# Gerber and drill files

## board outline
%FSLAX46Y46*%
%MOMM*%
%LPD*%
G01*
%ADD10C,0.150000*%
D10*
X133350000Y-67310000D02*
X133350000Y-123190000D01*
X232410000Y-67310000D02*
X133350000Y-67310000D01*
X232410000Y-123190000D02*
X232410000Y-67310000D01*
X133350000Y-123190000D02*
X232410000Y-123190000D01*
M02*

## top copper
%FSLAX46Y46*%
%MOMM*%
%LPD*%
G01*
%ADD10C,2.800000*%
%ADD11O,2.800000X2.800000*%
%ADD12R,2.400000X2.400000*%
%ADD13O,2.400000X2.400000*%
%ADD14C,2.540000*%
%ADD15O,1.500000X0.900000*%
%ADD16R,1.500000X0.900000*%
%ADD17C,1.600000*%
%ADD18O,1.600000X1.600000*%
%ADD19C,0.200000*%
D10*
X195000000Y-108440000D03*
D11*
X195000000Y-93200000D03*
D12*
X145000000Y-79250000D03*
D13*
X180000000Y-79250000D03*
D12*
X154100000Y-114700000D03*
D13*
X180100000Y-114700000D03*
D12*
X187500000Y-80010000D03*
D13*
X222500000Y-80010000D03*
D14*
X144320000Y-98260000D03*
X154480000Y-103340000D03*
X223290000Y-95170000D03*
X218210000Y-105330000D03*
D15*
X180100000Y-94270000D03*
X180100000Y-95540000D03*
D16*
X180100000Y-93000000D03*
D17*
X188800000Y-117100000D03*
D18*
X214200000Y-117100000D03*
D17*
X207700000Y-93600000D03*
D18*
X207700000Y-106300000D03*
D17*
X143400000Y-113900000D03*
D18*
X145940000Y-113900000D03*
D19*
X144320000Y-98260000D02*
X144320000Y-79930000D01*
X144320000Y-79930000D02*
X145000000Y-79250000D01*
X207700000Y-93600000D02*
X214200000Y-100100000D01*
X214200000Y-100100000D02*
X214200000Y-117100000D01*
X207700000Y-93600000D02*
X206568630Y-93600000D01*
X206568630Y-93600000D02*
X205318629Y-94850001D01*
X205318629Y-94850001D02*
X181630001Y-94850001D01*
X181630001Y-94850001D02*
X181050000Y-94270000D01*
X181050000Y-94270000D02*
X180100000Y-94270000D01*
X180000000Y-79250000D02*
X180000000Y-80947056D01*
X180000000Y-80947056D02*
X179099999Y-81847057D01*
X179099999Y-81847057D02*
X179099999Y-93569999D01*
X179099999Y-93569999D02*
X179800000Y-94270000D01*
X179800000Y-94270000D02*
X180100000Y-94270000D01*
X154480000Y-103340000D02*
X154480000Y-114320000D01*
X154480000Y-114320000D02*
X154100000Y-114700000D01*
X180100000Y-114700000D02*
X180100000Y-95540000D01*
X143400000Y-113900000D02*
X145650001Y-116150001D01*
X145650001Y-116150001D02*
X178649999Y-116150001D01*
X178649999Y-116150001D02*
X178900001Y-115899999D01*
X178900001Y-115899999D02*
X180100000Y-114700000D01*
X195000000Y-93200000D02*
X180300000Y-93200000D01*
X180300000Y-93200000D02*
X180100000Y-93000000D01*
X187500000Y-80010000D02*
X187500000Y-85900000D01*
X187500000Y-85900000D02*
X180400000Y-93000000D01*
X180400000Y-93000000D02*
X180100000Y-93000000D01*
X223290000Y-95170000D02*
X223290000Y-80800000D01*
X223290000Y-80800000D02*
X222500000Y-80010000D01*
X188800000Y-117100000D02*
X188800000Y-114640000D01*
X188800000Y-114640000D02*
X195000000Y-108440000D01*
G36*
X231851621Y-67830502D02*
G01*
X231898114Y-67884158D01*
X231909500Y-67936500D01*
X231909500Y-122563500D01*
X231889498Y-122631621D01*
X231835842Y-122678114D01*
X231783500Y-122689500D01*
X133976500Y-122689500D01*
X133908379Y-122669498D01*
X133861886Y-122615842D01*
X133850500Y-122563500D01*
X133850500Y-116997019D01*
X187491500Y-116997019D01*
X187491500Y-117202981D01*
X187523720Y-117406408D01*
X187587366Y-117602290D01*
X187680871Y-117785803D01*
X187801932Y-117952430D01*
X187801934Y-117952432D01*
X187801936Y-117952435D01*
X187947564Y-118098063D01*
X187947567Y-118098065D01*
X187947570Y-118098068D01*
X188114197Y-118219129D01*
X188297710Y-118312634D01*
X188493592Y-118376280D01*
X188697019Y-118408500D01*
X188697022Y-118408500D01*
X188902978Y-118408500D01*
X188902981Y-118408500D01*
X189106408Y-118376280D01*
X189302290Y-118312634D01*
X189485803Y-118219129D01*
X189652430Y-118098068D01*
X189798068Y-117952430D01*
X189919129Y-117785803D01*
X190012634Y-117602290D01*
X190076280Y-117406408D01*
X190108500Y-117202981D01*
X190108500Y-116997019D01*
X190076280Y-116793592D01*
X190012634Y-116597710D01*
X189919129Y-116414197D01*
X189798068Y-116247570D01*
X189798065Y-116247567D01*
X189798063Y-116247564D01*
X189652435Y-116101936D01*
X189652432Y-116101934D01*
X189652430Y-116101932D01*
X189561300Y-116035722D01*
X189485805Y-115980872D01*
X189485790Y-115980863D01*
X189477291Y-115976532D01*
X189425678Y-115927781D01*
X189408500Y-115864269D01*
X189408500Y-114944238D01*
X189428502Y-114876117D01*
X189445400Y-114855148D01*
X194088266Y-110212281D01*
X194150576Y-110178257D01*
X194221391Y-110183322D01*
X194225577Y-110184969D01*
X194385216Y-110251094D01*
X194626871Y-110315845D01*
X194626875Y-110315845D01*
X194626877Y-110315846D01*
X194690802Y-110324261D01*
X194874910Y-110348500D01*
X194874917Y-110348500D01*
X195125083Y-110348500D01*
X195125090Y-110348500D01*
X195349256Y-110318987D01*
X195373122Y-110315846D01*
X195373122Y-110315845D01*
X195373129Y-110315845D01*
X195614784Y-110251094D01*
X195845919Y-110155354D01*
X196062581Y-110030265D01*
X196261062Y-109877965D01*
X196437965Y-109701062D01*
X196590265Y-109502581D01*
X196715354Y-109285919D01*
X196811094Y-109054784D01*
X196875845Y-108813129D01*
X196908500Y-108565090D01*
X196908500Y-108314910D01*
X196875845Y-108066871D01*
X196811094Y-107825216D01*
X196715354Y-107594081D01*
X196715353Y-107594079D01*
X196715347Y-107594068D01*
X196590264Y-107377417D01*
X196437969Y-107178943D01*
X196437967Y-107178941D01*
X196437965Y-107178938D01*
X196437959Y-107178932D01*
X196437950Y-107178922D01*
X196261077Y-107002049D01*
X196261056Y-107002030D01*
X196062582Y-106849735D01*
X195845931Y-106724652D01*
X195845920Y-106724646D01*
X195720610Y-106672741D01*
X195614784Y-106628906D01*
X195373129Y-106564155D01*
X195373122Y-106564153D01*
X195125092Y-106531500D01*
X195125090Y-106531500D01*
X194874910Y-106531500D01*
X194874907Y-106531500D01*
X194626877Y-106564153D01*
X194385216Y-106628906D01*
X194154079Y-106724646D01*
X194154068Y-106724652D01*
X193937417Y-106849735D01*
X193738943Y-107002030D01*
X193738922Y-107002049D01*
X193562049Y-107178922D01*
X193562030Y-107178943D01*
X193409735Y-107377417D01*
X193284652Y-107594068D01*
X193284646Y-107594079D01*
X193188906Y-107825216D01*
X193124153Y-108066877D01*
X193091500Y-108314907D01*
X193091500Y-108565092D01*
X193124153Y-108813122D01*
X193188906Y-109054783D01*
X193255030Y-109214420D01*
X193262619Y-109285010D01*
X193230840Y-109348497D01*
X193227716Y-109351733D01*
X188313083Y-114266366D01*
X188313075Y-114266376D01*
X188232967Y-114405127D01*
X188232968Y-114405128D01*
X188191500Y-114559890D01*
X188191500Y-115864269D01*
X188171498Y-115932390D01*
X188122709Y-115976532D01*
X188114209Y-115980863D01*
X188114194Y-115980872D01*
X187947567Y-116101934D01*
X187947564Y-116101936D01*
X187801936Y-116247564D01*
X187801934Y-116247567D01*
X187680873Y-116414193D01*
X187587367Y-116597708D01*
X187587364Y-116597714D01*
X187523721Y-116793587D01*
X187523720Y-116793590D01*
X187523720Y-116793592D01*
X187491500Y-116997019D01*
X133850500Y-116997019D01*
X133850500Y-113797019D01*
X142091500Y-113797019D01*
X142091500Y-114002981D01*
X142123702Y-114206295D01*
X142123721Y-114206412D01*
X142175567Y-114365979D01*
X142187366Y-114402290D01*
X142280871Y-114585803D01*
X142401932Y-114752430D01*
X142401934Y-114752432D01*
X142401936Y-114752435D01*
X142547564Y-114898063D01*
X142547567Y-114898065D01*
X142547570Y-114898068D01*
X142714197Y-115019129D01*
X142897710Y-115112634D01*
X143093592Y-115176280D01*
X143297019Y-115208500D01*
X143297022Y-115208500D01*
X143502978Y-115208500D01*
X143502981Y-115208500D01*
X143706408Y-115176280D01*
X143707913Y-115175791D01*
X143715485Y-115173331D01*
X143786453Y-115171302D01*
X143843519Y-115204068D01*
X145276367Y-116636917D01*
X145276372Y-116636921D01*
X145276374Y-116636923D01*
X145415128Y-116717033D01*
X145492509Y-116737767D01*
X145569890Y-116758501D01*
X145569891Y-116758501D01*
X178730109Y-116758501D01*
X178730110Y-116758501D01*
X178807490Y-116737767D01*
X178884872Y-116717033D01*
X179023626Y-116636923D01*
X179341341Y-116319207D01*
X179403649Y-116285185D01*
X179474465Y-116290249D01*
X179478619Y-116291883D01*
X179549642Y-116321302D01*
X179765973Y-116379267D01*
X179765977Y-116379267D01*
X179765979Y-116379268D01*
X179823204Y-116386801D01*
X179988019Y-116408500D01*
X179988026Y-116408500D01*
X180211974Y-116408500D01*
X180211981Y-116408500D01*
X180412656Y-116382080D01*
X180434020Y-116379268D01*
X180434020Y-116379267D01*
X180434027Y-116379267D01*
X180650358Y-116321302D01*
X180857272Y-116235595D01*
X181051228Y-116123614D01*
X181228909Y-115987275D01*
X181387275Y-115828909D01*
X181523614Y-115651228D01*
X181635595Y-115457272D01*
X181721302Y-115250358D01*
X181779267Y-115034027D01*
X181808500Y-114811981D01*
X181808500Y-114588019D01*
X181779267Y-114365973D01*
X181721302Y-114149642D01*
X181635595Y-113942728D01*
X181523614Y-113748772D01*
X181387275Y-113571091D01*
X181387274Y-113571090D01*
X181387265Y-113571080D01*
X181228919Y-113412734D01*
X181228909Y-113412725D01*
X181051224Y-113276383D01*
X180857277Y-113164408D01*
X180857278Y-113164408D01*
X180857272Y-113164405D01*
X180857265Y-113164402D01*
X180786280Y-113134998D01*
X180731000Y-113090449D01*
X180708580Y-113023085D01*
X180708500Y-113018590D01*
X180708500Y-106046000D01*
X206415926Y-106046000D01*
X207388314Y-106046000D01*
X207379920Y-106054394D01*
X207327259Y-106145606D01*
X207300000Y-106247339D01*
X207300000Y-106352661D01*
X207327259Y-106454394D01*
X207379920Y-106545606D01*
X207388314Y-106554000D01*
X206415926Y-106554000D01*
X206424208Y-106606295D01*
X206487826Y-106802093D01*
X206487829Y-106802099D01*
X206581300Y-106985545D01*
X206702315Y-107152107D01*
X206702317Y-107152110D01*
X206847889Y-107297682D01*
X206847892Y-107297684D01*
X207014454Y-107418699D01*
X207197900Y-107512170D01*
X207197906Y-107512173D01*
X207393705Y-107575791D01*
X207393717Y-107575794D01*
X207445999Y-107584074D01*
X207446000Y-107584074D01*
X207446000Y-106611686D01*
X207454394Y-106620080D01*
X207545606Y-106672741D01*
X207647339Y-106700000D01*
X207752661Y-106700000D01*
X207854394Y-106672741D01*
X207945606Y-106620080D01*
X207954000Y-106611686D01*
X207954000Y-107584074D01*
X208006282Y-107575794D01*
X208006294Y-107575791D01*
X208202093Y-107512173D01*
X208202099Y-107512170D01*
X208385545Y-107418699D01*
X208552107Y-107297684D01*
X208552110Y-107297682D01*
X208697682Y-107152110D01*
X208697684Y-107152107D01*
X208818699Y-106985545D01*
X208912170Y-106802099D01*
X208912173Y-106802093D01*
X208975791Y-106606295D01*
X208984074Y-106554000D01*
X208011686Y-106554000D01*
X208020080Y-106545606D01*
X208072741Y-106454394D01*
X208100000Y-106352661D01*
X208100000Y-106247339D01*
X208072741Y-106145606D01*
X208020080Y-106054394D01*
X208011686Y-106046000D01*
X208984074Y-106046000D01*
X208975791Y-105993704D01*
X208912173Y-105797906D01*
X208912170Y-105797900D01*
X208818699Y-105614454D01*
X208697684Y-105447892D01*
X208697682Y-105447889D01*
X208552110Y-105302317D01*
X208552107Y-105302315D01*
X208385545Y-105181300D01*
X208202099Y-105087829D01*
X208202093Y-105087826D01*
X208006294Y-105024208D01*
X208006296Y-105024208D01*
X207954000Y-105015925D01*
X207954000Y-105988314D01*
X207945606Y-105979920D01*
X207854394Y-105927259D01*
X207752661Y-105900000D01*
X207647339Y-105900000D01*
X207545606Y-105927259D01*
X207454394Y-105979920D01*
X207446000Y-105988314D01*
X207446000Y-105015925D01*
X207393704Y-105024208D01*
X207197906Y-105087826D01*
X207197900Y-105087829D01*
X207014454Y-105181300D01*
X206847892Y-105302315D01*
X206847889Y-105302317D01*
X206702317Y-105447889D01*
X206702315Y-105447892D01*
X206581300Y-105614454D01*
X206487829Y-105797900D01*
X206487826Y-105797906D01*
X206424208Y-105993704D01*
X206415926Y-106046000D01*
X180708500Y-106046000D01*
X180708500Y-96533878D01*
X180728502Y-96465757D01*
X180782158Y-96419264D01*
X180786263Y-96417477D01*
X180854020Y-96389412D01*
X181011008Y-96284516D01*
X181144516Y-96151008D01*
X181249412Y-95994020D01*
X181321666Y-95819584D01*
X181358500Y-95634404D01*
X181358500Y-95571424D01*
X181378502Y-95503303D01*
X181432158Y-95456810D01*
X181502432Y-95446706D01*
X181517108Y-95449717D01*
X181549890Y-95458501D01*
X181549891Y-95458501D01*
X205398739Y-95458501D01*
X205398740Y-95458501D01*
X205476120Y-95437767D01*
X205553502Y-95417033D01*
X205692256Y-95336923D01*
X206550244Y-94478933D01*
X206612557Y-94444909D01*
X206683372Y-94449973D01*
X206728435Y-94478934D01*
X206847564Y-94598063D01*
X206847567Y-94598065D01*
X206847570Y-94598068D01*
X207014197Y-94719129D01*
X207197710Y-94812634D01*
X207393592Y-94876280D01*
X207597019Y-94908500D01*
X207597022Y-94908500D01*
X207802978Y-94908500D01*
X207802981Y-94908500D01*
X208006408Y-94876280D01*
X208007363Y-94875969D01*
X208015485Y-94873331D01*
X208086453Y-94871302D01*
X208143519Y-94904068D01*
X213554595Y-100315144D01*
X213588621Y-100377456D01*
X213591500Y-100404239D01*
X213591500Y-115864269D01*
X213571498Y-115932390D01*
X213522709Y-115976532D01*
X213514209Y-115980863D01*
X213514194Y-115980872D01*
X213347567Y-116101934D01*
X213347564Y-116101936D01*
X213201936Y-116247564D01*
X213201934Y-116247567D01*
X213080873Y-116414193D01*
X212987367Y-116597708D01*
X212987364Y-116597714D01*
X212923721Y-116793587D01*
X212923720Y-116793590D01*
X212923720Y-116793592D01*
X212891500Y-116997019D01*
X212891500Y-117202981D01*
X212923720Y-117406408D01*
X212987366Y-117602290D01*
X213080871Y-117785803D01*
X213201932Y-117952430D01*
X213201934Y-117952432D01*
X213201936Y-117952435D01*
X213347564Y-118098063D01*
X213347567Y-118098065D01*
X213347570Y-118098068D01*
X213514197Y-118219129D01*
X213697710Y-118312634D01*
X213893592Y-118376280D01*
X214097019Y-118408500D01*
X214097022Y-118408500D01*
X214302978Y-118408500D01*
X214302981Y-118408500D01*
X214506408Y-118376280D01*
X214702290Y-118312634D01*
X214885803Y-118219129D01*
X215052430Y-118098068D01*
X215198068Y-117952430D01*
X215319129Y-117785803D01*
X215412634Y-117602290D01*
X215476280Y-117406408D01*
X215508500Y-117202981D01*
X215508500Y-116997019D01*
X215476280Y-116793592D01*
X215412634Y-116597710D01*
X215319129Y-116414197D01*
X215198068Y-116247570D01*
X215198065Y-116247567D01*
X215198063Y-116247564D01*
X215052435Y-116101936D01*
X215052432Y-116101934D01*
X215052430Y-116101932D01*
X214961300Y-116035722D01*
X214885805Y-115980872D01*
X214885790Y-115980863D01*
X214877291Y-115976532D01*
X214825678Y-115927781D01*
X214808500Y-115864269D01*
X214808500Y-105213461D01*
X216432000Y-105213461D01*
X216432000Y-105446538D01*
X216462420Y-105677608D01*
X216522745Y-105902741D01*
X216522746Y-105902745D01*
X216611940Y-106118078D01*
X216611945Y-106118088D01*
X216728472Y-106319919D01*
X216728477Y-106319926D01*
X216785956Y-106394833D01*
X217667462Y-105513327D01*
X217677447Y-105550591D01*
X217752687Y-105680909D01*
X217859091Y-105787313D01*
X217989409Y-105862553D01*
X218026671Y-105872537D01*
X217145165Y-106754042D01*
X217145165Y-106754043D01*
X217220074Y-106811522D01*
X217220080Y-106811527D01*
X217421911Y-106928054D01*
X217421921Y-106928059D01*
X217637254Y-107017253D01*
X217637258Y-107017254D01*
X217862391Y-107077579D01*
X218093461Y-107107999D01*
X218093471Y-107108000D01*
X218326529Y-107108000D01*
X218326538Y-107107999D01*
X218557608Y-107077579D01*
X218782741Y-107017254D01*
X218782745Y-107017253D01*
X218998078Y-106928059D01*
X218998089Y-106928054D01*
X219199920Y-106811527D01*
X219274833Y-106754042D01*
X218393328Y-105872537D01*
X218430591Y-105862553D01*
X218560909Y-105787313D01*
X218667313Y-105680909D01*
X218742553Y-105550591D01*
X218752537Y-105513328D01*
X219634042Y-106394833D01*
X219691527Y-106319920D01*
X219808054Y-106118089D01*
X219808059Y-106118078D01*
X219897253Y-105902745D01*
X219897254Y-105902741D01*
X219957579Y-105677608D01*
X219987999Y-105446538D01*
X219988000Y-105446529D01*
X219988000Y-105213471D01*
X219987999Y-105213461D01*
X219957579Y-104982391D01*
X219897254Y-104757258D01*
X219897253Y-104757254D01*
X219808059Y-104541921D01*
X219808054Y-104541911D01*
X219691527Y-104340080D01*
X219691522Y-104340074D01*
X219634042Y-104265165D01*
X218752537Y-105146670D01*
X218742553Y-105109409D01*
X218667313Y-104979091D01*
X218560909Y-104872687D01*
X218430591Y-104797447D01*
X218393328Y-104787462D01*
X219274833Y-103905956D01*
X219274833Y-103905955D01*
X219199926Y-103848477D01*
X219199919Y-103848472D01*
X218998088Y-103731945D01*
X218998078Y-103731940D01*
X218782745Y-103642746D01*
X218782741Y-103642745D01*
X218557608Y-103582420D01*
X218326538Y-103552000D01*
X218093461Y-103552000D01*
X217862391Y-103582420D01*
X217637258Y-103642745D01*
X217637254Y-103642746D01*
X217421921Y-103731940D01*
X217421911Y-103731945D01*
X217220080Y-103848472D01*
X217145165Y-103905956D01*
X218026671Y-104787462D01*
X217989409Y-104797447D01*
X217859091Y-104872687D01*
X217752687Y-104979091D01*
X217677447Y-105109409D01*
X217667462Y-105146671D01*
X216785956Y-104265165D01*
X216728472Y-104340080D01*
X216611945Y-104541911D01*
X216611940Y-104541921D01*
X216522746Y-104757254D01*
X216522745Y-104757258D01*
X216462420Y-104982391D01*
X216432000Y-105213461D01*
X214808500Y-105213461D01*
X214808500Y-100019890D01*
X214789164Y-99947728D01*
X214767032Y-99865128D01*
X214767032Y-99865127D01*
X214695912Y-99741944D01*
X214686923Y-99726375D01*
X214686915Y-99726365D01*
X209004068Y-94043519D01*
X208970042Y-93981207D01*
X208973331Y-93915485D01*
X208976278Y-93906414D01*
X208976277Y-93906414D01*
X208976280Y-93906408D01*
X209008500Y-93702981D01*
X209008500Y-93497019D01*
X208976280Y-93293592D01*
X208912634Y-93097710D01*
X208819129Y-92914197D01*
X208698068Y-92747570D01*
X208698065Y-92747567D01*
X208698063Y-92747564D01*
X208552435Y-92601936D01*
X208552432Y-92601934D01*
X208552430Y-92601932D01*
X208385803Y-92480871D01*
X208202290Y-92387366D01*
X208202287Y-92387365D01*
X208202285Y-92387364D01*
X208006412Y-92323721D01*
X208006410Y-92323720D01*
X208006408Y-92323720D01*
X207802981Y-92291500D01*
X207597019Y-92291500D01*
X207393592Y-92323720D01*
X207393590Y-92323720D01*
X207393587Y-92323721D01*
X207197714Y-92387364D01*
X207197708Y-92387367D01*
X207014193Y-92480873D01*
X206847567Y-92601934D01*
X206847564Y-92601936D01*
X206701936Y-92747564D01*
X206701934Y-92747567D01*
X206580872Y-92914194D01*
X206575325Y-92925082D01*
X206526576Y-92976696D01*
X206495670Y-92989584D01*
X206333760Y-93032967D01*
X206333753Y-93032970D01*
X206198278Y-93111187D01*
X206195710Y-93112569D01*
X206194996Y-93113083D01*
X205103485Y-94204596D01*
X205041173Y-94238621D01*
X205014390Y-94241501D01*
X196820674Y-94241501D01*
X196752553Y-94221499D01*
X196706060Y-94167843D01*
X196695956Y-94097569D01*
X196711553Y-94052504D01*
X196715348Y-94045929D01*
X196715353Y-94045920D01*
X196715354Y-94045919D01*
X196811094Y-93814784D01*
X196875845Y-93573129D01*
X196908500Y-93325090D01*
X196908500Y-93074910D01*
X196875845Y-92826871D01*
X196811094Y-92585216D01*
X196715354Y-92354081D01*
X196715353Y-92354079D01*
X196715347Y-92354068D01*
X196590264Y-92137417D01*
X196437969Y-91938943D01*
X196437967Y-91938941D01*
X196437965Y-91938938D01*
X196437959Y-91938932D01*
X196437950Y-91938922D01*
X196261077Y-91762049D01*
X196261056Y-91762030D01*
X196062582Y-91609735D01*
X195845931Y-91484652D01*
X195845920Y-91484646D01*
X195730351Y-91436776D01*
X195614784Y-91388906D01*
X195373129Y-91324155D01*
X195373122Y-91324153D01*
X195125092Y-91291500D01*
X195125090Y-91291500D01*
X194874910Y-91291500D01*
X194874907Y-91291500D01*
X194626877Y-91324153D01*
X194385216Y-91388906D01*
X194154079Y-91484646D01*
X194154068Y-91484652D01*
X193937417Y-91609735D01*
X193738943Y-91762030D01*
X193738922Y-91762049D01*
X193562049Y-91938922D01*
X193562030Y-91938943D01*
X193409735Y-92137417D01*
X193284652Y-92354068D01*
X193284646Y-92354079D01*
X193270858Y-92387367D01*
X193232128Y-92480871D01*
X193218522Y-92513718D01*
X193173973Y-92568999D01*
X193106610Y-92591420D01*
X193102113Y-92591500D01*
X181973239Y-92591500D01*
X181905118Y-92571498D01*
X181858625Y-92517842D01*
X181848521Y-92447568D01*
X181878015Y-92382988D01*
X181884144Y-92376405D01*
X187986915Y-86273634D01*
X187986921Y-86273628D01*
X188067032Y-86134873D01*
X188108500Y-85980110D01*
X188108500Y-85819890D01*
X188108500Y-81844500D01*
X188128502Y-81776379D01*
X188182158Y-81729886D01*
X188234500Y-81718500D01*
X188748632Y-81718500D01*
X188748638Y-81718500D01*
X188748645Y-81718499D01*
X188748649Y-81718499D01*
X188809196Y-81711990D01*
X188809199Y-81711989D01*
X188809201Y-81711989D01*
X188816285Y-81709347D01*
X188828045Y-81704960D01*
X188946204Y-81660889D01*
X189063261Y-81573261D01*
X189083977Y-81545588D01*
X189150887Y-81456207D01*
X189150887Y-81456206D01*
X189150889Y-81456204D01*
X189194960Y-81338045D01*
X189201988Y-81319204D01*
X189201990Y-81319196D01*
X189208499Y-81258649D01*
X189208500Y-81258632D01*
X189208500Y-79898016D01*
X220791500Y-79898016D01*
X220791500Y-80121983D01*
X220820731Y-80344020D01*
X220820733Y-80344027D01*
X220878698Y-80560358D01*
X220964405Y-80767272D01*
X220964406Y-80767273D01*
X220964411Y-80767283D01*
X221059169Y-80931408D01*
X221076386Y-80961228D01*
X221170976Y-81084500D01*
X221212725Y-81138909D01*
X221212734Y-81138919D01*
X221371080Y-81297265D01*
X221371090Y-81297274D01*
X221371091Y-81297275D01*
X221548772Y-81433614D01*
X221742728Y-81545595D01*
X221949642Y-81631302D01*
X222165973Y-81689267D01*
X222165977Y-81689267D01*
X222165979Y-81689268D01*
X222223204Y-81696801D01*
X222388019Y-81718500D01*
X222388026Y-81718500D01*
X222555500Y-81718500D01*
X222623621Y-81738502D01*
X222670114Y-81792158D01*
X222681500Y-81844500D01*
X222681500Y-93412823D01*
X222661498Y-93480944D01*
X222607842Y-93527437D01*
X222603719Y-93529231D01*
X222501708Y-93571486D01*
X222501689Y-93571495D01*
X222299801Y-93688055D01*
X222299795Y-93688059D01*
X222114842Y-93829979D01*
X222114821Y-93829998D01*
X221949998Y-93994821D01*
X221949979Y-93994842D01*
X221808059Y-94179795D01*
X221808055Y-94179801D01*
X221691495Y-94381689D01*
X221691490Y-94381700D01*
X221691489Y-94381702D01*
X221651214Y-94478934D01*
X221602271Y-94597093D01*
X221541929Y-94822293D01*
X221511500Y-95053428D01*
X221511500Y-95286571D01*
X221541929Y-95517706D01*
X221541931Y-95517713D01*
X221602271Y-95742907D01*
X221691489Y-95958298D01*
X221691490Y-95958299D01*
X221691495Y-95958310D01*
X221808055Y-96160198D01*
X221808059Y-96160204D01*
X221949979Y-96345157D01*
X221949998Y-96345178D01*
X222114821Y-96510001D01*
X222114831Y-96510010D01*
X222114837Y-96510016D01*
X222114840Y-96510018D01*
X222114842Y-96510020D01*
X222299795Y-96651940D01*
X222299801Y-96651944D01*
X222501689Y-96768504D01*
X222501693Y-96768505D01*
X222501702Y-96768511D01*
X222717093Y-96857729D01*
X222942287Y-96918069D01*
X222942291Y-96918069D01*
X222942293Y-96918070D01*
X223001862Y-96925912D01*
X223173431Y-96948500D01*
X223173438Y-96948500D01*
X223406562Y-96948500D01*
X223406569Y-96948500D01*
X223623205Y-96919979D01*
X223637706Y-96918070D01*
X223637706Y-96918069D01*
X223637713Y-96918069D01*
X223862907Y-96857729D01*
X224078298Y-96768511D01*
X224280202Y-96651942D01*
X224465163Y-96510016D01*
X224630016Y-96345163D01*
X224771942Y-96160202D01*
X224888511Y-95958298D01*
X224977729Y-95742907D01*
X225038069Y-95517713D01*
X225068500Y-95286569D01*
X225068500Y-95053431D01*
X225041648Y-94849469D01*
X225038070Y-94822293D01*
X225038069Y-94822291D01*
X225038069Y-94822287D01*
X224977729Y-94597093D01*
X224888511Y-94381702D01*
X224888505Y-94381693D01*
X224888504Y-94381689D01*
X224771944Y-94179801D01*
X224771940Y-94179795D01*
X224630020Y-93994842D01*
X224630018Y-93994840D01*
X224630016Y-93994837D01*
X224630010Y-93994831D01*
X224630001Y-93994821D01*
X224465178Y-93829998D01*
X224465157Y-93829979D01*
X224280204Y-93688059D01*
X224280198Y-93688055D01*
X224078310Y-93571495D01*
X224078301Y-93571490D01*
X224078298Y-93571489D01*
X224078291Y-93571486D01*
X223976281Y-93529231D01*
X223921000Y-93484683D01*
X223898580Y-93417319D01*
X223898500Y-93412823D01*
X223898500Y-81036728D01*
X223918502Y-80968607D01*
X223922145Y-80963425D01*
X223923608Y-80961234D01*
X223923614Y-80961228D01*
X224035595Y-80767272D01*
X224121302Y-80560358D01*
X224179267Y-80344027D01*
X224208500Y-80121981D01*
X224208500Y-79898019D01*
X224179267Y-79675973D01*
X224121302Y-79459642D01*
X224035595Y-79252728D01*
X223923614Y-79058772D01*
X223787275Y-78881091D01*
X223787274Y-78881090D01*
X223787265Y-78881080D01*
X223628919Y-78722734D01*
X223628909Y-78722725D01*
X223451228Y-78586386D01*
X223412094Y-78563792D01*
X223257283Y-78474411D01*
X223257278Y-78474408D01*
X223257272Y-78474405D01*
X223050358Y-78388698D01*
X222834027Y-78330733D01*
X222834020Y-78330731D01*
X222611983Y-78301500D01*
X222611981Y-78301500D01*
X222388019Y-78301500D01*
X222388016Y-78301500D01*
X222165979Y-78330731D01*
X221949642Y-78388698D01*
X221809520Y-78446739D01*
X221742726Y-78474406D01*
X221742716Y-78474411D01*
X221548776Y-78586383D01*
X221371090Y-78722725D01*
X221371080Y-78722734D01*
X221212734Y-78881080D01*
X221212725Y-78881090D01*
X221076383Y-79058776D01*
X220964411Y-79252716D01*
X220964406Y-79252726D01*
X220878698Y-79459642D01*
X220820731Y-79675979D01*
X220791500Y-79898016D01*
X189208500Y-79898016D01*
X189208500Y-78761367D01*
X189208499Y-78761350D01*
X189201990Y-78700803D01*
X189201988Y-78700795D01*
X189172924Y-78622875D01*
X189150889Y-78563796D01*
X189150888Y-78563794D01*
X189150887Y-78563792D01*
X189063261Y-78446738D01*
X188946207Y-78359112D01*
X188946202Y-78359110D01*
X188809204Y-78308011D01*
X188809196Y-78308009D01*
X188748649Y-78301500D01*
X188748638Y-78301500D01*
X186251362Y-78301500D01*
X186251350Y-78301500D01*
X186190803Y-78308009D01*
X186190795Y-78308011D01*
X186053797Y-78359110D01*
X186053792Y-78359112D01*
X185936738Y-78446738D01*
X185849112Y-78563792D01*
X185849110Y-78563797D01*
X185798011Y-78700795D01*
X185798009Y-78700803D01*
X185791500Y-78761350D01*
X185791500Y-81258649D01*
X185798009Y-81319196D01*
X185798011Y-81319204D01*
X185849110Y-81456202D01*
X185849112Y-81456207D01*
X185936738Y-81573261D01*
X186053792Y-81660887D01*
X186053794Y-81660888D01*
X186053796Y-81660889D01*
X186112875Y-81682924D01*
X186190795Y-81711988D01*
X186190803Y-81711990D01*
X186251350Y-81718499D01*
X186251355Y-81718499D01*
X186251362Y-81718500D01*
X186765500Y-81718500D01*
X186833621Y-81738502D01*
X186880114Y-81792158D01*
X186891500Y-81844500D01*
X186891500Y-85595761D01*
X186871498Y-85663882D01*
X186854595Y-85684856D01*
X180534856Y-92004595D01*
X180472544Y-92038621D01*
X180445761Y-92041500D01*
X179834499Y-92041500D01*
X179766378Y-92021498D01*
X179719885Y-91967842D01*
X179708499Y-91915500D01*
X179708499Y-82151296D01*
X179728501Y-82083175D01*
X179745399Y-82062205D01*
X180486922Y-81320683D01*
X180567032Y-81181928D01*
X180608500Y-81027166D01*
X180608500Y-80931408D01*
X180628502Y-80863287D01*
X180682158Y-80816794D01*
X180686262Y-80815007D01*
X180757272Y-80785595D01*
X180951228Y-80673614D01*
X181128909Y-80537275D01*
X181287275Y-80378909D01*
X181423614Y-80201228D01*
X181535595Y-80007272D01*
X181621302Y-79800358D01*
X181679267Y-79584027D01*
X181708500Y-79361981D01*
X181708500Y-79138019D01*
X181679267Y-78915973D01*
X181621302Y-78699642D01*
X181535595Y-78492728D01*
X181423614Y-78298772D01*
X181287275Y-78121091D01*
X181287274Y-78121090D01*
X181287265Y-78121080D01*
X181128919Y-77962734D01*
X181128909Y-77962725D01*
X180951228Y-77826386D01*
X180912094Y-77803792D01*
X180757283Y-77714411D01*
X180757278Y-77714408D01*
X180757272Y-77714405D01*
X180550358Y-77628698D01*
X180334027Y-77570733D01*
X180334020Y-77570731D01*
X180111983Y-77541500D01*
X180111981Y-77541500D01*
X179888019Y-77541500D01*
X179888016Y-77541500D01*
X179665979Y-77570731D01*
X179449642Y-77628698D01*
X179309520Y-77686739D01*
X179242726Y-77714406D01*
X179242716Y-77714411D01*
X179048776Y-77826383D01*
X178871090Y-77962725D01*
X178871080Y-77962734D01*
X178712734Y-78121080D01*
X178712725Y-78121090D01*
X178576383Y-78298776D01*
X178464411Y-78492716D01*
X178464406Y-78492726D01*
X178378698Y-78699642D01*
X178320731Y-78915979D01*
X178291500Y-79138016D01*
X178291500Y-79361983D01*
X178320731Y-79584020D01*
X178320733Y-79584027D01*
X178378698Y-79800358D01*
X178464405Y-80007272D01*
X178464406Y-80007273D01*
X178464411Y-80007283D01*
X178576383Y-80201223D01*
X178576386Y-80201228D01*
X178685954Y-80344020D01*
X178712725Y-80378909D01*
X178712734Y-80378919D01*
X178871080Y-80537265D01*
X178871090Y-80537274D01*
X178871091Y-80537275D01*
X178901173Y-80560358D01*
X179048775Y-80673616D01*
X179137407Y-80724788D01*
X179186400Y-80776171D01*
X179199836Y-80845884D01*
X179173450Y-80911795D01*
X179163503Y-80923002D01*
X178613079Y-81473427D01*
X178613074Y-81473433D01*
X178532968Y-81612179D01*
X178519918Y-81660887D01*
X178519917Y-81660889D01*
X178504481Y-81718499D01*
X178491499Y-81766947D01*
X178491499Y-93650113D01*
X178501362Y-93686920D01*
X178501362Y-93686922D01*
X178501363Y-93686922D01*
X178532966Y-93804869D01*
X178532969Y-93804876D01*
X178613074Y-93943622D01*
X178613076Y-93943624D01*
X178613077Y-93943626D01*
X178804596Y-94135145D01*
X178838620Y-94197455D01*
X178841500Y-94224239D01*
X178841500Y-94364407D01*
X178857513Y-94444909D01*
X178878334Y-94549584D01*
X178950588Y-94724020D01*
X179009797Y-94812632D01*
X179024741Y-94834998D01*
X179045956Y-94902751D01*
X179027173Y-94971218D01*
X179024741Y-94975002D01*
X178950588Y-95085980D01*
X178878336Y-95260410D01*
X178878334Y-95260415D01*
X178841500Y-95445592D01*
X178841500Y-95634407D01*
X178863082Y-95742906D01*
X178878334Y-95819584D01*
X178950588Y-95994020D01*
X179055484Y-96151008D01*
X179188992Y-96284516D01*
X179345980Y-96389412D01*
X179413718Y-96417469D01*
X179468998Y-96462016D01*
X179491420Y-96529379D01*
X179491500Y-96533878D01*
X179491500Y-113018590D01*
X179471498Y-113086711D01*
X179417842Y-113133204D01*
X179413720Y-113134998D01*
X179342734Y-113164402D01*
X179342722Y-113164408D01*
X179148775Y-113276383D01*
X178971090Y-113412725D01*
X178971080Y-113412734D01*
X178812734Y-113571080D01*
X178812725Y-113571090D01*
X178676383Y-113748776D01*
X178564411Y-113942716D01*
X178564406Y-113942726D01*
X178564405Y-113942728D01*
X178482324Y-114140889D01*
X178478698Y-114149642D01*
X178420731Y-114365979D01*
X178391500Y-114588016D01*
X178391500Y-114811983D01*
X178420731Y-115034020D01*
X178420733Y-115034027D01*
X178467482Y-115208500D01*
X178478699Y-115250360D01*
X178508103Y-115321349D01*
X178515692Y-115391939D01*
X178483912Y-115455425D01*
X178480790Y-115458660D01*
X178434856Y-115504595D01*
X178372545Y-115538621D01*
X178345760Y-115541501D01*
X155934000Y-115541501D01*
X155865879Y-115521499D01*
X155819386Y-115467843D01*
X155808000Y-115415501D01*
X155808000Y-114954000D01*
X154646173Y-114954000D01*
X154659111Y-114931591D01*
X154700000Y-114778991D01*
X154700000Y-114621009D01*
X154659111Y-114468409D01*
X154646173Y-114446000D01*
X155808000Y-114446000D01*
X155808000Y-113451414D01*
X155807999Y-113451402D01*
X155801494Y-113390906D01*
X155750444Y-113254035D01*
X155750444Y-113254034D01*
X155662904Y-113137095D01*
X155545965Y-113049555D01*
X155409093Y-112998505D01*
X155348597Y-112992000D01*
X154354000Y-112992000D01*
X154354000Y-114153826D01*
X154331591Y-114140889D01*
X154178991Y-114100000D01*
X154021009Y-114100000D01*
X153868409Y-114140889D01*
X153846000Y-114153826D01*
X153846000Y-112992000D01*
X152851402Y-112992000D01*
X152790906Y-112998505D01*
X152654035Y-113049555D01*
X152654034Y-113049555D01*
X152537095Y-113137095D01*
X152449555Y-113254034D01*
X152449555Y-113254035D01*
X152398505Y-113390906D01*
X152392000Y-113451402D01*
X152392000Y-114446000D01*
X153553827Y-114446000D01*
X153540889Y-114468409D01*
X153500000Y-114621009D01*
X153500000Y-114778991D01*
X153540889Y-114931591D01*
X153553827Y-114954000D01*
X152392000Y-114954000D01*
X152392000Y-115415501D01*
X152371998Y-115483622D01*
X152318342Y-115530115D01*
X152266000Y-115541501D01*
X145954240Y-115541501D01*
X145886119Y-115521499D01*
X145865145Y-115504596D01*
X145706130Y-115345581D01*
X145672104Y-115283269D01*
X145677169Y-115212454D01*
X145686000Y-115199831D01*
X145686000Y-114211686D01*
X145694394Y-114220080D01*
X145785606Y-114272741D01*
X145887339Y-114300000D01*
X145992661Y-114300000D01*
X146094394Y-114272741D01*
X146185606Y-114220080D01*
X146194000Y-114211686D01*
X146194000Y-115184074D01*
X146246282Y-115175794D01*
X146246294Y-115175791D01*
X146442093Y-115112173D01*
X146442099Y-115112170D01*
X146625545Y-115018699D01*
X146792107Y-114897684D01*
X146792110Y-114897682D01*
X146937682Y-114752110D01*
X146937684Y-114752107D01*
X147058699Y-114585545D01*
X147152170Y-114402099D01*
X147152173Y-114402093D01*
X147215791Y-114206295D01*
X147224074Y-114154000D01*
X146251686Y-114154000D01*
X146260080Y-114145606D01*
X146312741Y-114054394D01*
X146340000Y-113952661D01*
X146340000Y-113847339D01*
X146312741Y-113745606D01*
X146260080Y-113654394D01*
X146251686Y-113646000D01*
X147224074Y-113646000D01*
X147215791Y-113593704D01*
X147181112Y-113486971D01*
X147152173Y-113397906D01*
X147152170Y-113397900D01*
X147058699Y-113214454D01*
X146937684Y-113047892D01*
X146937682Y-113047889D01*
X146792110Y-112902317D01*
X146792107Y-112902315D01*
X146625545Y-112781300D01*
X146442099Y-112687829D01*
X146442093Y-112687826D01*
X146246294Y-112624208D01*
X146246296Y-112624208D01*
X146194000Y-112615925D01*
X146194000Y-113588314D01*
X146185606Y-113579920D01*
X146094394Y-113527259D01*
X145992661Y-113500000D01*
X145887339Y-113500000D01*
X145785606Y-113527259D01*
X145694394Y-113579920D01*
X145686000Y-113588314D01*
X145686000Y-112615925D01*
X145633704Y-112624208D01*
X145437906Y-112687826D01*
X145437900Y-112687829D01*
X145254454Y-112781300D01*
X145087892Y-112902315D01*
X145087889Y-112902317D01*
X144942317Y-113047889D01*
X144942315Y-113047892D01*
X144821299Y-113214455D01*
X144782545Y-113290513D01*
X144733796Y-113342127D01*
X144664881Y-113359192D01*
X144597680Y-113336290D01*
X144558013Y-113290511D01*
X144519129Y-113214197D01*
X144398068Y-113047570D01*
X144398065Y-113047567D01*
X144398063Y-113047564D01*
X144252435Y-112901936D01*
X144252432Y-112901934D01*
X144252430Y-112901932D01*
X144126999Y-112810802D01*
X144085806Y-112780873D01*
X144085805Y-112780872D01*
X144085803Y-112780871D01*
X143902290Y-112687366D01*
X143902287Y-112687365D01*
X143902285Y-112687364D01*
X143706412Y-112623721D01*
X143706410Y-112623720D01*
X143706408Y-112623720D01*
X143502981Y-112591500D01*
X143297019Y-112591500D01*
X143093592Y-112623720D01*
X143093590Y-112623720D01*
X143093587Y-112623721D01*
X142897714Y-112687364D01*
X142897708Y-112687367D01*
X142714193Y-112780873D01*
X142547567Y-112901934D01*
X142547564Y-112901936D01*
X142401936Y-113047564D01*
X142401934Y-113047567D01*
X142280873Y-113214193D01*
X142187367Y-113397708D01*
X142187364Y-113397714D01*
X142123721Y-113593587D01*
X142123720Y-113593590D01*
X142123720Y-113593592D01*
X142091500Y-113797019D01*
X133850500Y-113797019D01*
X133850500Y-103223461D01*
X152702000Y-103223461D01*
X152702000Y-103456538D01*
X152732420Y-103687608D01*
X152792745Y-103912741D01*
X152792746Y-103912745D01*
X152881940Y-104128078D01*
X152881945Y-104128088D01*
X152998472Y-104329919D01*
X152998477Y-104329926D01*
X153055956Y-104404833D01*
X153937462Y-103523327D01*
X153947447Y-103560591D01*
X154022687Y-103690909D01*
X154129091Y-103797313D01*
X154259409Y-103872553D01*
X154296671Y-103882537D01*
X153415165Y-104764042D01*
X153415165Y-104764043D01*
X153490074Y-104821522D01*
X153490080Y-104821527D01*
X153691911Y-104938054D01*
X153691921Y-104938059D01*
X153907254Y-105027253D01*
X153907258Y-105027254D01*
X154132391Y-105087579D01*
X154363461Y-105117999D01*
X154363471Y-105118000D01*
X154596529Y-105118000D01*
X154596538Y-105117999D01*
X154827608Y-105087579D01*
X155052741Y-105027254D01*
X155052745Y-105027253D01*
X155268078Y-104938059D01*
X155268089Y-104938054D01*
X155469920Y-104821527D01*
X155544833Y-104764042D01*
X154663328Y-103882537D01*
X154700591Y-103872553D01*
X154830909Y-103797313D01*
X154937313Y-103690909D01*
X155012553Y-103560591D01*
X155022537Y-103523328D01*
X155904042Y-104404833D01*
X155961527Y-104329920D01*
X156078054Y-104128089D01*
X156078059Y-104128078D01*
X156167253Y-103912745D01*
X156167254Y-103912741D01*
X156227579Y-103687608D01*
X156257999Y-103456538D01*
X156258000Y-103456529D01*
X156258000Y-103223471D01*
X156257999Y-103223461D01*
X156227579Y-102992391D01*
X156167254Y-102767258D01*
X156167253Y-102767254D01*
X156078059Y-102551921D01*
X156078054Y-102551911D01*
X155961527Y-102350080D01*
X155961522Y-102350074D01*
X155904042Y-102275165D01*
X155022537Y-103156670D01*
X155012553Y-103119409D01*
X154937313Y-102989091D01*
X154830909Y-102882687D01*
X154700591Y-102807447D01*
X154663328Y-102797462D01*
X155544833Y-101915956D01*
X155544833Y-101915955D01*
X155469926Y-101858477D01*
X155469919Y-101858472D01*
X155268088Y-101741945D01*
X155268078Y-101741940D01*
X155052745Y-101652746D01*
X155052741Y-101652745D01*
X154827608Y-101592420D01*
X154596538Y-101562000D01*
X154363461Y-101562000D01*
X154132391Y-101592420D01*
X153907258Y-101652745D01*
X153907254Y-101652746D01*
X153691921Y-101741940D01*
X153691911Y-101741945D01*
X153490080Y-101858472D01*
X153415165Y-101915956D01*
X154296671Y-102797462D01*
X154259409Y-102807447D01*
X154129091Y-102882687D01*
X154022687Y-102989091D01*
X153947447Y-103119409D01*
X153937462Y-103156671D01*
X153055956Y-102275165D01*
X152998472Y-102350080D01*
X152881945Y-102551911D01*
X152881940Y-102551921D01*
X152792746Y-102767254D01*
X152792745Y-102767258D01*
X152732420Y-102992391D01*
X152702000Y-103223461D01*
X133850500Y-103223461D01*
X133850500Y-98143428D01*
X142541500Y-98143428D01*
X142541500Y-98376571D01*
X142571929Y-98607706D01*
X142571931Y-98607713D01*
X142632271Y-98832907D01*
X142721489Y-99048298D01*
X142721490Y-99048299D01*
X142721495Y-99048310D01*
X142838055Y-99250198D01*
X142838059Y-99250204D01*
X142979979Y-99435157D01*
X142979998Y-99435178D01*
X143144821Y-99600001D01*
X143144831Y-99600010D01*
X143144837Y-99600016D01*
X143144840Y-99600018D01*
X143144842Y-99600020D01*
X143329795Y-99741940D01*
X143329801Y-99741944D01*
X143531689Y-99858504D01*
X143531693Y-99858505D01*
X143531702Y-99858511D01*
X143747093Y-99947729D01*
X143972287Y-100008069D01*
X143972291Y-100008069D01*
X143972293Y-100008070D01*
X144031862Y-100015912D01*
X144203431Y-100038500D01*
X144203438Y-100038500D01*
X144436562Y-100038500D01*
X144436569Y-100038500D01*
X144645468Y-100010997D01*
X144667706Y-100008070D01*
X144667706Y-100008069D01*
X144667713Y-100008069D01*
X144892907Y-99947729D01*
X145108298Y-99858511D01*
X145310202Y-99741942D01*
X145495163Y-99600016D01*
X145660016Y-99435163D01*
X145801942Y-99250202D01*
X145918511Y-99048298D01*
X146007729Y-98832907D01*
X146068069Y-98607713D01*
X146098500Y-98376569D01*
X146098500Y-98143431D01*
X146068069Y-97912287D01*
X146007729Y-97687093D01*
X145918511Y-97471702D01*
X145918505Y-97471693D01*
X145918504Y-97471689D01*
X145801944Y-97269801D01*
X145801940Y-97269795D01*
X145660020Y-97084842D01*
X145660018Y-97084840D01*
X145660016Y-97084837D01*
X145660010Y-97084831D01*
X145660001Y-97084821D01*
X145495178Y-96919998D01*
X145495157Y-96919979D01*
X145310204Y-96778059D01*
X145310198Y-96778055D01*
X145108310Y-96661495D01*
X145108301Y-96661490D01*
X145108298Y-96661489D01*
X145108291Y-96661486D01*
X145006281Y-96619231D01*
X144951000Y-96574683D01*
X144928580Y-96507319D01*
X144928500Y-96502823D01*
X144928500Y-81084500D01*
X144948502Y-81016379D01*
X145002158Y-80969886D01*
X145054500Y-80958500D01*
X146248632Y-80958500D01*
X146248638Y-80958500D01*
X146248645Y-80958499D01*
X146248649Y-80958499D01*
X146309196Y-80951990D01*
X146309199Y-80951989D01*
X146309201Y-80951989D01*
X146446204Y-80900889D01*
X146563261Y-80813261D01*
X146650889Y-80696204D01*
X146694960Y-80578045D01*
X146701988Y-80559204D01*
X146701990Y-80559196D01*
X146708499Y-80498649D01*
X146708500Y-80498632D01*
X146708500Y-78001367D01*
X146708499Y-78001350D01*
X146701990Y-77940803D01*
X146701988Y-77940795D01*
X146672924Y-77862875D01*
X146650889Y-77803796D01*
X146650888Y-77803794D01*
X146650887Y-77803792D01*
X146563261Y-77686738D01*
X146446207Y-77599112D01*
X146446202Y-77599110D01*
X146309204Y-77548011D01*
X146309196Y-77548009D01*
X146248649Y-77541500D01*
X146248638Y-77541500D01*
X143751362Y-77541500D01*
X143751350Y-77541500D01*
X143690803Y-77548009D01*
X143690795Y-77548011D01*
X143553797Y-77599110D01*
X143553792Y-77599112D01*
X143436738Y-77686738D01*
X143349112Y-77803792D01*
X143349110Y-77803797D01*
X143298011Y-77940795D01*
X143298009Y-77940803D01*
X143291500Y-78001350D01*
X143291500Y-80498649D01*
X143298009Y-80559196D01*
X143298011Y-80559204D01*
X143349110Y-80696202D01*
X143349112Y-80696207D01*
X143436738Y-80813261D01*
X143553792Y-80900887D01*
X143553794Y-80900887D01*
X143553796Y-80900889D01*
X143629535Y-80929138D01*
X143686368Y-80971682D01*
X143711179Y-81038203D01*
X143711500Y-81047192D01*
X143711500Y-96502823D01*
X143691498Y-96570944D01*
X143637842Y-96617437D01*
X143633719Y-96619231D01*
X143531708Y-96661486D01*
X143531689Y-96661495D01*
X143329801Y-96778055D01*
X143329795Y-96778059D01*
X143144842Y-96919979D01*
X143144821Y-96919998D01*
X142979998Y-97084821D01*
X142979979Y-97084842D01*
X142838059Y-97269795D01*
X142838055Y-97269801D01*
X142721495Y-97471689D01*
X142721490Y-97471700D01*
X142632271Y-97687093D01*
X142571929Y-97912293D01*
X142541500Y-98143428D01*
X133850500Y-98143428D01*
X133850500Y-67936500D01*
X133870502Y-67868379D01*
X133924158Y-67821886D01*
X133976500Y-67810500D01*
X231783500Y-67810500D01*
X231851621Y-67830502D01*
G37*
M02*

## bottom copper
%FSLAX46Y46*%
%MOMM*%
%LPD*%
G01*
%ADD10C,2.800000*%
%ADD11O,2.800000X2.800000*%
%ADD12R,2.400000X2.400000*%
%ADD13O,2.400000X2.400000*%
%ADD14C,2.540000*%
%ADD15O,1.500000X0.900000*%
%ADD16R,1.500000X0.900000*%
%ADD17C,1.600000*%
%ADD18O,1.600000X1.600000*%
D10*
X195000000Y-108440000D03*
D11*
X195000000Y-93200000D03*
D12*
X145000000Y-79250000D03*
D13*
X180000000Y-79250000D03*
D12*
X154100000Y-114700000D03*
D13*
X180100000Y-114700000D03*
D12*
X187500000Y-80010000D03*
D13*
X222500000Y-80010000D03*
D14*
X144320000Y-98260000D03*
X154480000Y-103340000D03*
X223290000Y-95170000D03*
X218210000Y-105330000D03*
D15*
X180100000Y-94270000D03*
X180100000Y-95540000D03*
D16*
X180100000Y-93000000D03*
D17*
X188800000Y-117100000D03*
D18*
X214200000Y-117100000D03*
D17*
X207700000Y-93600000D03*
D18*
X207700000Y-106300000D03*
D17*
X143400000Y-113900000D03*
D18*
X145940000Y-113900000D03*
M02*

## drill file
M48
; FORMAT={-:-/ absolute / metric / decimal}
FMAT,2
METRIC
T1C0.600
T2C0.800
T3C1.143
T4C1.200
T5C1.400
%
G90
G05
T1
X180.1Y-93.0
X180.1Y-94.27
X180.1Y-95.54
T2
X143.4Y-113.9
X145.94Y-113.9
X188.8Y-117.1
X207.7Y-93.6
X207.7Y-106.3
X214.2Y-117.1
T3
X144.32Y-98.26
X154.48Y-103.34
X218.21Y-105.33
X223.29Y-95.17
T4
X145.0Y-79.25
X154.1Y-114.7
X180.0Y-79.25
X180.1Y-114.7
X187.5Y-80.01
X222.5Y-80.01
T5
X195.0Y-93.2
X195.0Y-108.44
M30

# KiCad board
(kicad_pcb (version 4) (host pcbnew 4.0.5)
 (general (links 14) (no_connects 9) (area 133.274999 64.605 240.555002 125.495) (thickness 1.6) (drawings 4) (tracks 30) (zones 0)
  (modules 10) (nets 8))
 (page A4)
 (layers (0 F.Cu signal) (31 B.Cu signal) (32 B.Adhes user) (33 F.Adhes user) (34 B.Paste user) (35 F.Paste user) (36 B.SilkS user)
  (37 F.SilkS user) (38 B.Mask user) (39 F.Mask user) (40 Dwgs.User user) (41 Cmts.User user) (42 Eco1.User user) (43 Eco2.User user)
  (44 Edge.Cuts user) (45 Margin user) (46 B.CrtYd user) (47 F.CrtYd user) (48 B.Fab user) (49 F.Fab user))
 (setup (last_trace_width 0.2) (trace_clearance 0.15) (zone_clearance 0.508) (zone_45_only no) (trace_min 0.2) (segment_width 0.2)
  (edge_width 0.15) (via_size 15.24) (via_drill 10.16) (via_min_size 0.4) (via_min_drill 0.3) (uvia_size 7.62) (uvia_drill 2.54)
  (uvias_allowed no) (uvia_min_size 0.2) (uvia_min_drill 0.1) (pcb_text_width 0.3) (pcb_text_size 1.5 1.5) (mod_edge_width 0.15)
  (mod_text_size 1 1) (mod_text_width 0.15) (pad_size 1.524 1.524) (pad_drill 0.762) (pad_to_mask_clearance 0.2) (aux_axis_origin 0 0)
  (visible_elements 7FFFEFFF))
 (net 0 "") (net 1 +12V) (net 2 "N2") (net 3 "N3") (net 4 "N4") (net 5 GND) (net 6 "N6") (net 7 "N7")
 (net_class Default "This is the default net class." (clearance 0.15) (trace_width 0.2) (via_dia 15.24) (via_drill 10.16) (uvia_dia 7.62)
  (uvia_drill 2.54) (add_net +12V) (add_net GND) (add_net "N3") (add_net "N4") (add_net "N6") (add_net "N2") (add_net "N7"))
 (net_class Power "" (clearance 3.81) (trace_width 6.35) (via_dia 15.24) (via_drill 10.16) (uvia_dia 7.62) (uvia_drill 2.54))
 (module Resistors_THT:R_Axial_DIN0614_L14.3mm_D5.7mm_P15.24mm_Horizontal (layer F.Cu) (at 195 108.44 90)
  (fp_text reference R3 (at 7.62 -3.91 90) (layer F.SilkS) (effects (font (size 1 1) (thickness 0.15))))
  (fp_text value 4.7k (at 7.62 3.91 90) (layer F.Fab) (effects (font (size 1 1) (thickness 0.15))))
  (pad 1 thru_hole circle (at 0 0 90) (size 2.8 2.8) (drill 1.4) (layers *.Cu *.Mask) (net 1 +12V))
  (pad 2 thru_hole oval (at 15.24 0 90) (size 2.8 2.8) (drill 1.4) (layers *.Cu *.Mask) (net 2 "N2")))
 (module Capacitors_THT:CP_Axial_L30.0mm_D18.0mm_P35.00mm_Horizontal (layer F.Cu) (at 145 79.25)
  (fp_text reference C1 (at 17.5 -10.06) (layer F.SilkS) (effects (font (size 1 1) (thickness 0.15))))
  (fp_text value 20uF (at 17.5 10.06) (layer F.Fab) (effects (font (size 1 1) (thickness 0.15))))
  (pad 1 thru_hole rect (at 0 0) (size 2.4 2.4) (drill 1.2) (layers *.Cu *.Mask) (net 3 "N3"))
  (pad 2 thru_hole oval (at 35 0) (size 2.4 2.4) (drill 1.2) (layers *.Cu *.Mask) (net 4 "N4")))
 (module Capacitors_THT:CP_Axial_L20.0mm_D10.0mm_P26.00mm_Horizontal (layer F.Cu) (at 154.1 114.7)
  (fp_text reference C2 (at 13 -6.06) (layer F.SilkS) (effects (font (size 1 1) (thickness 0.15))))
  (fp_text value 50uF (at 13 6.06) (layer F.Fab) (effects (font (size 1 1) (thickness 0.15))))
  (pad 1 thru_hole rect (at 0 0) (size 2.4 2.4) (drill 1.2) (layers *.Cu *.Mask) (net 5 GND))
  (pad 2 thru_hole oval (at 26 0) (size 2.4 2.4) (drill 1.2) (layers *.Cu *.Mask) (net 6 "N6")))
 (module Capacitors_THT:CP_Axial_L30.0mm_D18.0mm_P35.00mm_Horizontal (layer F.Cu) (at 187.5 80.01)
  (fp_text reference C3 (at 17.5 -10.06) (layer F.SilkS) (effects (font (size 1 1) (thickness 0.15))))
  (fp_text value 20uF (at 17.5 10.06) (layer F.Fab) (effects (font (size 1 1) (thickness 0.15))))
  (pad 1 thru_hole rect (at 0 0) (size 2.4 2.4) (drill 1.2) (layers *.Cu *.Mask) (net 2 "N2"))
  (pad 2 thru_hole oval (at 35 0) (size 2.4 2.4) (drill 1.2) (layers *.Cu *.Mask) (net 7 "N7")))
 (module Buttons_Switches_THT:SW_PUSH (layer F.Cu) (at 149.4 100.8)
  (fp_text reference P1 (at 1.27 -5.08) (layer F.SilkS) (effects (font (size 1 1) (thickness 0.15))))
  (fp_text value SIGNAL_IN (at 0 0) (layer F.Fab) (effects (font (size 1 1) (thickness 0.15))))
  (pad 1 thru_hole circle (at -5.08 -2.54) (size 2.54 2.54) (drill 1.143) (layers *.Cu *.Mask) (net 3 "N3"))
  (pad 2 thru_hole circle (at 5.08 2.54) (size 2.54 2.54) (drill 1.143) (layers *.Cu *.Mask) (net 5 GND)))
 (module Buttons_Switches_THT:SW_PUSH (layer F.Cu) (at 220.75 100.25 270)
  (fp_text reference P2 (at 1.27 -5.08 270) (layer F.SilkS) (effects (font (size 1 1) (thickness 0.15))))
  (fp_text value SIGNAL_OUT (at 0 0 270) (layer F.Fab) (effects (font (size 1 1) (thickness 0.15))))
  (pad 1 thru_hole circle (at -5.08 -2.54 270) (size 2.54 2.54) (drill 1.143) (layers *.Cu *.Mask) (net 7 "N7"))
  (pad 2 thru_hole circle (at 5.08 2.54 270) (size 2.54 2.54) (drill 1.143) (layers *.Cu *.Mask) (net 5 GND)))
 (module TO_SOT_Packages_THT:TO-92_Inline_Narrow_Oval (layer F.Cu) (at 180.1 93 270)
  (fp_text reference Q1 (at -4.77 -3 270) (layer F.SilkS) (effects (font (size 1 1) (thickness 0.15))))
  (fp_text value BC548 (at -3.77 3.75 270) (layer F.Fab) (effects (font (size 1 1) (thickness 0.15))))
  (pad 2 thru_hole oval (at 1.27 0 90) (size 0.9 1.5) (drill 0.6) (layers *.Cu *.Mask) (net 4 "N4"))
  (pad 3 thru_hole oval (at 2.54 0 90) (size 0.9 1.5) (drill 0.6) (layers *.Cu *.Mask) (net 6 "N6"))
  (pad 1 thru_hole rect (at 0 0 90) (size 0.9 1.5) (drill 0.6) (layers *.Cu *.Mask) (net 2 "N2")))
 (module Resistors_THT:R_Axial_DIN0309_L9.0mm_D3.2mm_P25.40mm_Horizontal (layer F.Cu) (at 188.8 117.1)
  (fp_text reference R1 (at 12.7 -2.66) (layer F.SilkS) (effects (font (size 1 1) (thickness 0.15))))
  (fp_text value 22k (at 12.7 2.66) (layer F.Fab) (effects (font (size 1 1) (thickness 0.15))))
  (pad 1 thru_hole circle (at 0 0) (size 1.6 1.6) (drill 0.8) (layers *.Cu *.Mask) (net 1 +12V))
  (pad 2 thru_hole oval (at 25.4 0) (size 1.6 1.6) (drill 0.8) (layers *.Cu *.Mask) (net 4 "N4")))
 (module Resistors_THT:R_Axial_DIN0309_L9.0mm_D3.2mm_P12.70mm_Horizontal (layer F.Cu) (at 207.7 93.6 270)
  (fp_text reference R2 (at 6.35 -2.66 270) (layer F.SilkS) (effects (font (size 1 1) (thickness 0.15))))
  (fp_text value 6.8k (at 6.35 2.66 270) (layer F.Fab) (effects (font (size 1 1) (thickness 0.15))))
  (pad 1 thru_hole circle (at 0 0 270) (size 1.6 1.6) (drill 0.8) (layers *.Cu *.Mask) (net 4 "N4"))
  (pad 2 thru_hole oval (at 12.7 0 270) (size 1.6 1.6) (drill 0.8) (layers *.Cu *.Mask) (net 5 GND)))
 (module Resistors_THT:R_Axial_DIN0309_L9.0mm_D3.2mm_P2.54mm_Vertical (layer F.Cu) (at 143.4 113.9)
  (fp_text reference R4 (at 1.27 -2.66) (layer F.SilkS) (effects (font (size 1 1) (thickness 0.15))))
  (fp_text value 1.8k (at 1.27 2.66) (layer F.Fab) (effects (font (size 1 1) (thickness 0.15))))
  (pad 1 thru_hole circle (at 0 0) (size 1.6 1.6) (drill 0.8) (layers *.Cu *.Mask) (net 6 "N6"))
  (pad 2 thru_hole oval (at 2.54 0) (size 1.6 1.6) (drill 0.8) (layers *.Cu *.Mask) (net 5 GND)))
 (gr_line (start 133.35 67.31) (end 133.35 123.19) (layer Edge.Cuts) (width 0.15))
 (gr_line (start 232.41 67.31) (end 133.35 67.31) (layer Edge.Cuts) (width 0.15))
 (gr_line (start 232.41 123.19) (end 232.41 67.31) (layer Edge.Cuts) (width 0.15))
 (gr_line (start 133.35 123.19) (end 232.41 123.19) (layer Edge.Cuts) (width 0.15))
 (segment (start 144.32 98.26) (end 144.32 79.93) (width 0.2) (layer F.Cu) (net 3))
 (segment (start 144.32 79.93) (end 145 79.25) (width 0.2) (layer F.Cu) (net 3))
 (segment (start 207.7 93.6) (end 214.2 100.1) (width 0.2) (layer F.Cu) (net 4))
 (segment (start 214.2 100.1) (end 214.2 117.1) (width 0.2) (layer F.Cu) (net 4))
 (segment (start 207.7 93.6) (end 206.56863 93.6) (width 0.2) (layer F.Cu) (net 4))
 (segment (start 206.56863 93.6) (end 205.318629 94.850001) (width 0.2) (layer F.Cu) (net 4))
 (segment (start 205.318629 94.850001) (end 181.630001 94.850001) (width 0.2) (layer F.Cu) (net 4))
 (segment (start 181.630001 94.850001) (end 181.05 94.27) (width 0.2) (layer F.Cu) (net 4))
 (segment (start 181.05 94.27) (end 180.1 94.27) (width 0.2) (layer F.Cu) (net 4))
 (segment (start 180 79.25) (end 180 80.947056) (width 0.2) (layer F.Cu) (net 4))
 (segment (start 180 80.947056) (end 179.099999 81.847057) (width 0.2) (layer F.Cu) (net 4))
 (segment (start 179.099999 81.847057) (end 179.099999 93.569999) (width 0.2) (layer F.Cu) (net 4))
 (segment (start 179.099999 93.569999) (end 179.8 94.27) (width 0.2) (layer F.Cu) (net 4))
 (segment (start 179.8 94.27) (end 180.1 94.27) (width 0.2) (layer F.Cu) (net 4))
 (segment (start 154.48 103.34) (end 154.48 114.32) (width 0.2) (layer F.Cu) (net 5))
 (segment (start 154.48 114.32) (end 154.1 114.7) (width 0.2) (layer F.Cu) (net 5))
 (segment (start 180.1 114.7) (end 180.1 95.54) (width 0.2) (layer F.Cu) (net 6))
 (segment (start 143.4 113.9) (end 145.650001 116.150001) (width 0.2) (layer F.Cu) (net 6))
 (segment (start 145.650001 116.150001) (end 178.649999 116.150001) (width 0.2) (layer F.Cu) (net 6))
 (segment (start 178.649999 116.150001) (end 178.900001 115.899999) (width 0.2) (layer F.Cu) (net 6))
 (segment (start 178.900001 115.899999) (end 180.1 114.7) (width 0.2) (layer F.Cu) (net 6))
 (segment (start 195 93.2) (end 180.3 93.2) (width 0.2) (layer F.Cu) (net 2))
 (segment (start 180.3 93.2) (end 180.1 93) (width 0.2) (layer F.Cu) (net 2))
 (segment (start 187.5 80.01) (end 187.5 85.9) (width 0.2) (layer F.Cu) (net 2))
 (segment (start 187.5 85.9) (end 180.4 93) (width 0.2) (layer F.Cu) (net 2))
 (segment (start 180.4 93) (end 180.1 93) (width 0.2) (layer F.Cu) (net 2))
 (segment (start 223.29 95.17) (end 223.29 80.8) (width 0.2) (layer F.Cu) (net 7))
 (segment (start 223.29 80.8) (end 222.5 80.01) (width 0.2) (layer F.Cu) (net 7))
 (segment (start 188.8 117.1) (end 188.8 114.64) (width 0.2) (layer F.Cu) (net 1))
 (segment (start 188.8 114.64) (end 195 108.44) (width 0.2) (layer F.Cu) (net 1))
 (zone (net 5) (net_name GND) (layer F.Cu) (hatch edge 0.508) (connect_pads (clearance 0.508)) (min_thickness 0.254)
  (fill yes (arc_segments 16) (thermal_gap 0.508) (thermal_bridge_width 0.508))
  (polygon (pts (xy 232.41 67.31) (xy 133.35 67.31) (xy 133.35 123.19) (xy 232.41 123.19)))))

